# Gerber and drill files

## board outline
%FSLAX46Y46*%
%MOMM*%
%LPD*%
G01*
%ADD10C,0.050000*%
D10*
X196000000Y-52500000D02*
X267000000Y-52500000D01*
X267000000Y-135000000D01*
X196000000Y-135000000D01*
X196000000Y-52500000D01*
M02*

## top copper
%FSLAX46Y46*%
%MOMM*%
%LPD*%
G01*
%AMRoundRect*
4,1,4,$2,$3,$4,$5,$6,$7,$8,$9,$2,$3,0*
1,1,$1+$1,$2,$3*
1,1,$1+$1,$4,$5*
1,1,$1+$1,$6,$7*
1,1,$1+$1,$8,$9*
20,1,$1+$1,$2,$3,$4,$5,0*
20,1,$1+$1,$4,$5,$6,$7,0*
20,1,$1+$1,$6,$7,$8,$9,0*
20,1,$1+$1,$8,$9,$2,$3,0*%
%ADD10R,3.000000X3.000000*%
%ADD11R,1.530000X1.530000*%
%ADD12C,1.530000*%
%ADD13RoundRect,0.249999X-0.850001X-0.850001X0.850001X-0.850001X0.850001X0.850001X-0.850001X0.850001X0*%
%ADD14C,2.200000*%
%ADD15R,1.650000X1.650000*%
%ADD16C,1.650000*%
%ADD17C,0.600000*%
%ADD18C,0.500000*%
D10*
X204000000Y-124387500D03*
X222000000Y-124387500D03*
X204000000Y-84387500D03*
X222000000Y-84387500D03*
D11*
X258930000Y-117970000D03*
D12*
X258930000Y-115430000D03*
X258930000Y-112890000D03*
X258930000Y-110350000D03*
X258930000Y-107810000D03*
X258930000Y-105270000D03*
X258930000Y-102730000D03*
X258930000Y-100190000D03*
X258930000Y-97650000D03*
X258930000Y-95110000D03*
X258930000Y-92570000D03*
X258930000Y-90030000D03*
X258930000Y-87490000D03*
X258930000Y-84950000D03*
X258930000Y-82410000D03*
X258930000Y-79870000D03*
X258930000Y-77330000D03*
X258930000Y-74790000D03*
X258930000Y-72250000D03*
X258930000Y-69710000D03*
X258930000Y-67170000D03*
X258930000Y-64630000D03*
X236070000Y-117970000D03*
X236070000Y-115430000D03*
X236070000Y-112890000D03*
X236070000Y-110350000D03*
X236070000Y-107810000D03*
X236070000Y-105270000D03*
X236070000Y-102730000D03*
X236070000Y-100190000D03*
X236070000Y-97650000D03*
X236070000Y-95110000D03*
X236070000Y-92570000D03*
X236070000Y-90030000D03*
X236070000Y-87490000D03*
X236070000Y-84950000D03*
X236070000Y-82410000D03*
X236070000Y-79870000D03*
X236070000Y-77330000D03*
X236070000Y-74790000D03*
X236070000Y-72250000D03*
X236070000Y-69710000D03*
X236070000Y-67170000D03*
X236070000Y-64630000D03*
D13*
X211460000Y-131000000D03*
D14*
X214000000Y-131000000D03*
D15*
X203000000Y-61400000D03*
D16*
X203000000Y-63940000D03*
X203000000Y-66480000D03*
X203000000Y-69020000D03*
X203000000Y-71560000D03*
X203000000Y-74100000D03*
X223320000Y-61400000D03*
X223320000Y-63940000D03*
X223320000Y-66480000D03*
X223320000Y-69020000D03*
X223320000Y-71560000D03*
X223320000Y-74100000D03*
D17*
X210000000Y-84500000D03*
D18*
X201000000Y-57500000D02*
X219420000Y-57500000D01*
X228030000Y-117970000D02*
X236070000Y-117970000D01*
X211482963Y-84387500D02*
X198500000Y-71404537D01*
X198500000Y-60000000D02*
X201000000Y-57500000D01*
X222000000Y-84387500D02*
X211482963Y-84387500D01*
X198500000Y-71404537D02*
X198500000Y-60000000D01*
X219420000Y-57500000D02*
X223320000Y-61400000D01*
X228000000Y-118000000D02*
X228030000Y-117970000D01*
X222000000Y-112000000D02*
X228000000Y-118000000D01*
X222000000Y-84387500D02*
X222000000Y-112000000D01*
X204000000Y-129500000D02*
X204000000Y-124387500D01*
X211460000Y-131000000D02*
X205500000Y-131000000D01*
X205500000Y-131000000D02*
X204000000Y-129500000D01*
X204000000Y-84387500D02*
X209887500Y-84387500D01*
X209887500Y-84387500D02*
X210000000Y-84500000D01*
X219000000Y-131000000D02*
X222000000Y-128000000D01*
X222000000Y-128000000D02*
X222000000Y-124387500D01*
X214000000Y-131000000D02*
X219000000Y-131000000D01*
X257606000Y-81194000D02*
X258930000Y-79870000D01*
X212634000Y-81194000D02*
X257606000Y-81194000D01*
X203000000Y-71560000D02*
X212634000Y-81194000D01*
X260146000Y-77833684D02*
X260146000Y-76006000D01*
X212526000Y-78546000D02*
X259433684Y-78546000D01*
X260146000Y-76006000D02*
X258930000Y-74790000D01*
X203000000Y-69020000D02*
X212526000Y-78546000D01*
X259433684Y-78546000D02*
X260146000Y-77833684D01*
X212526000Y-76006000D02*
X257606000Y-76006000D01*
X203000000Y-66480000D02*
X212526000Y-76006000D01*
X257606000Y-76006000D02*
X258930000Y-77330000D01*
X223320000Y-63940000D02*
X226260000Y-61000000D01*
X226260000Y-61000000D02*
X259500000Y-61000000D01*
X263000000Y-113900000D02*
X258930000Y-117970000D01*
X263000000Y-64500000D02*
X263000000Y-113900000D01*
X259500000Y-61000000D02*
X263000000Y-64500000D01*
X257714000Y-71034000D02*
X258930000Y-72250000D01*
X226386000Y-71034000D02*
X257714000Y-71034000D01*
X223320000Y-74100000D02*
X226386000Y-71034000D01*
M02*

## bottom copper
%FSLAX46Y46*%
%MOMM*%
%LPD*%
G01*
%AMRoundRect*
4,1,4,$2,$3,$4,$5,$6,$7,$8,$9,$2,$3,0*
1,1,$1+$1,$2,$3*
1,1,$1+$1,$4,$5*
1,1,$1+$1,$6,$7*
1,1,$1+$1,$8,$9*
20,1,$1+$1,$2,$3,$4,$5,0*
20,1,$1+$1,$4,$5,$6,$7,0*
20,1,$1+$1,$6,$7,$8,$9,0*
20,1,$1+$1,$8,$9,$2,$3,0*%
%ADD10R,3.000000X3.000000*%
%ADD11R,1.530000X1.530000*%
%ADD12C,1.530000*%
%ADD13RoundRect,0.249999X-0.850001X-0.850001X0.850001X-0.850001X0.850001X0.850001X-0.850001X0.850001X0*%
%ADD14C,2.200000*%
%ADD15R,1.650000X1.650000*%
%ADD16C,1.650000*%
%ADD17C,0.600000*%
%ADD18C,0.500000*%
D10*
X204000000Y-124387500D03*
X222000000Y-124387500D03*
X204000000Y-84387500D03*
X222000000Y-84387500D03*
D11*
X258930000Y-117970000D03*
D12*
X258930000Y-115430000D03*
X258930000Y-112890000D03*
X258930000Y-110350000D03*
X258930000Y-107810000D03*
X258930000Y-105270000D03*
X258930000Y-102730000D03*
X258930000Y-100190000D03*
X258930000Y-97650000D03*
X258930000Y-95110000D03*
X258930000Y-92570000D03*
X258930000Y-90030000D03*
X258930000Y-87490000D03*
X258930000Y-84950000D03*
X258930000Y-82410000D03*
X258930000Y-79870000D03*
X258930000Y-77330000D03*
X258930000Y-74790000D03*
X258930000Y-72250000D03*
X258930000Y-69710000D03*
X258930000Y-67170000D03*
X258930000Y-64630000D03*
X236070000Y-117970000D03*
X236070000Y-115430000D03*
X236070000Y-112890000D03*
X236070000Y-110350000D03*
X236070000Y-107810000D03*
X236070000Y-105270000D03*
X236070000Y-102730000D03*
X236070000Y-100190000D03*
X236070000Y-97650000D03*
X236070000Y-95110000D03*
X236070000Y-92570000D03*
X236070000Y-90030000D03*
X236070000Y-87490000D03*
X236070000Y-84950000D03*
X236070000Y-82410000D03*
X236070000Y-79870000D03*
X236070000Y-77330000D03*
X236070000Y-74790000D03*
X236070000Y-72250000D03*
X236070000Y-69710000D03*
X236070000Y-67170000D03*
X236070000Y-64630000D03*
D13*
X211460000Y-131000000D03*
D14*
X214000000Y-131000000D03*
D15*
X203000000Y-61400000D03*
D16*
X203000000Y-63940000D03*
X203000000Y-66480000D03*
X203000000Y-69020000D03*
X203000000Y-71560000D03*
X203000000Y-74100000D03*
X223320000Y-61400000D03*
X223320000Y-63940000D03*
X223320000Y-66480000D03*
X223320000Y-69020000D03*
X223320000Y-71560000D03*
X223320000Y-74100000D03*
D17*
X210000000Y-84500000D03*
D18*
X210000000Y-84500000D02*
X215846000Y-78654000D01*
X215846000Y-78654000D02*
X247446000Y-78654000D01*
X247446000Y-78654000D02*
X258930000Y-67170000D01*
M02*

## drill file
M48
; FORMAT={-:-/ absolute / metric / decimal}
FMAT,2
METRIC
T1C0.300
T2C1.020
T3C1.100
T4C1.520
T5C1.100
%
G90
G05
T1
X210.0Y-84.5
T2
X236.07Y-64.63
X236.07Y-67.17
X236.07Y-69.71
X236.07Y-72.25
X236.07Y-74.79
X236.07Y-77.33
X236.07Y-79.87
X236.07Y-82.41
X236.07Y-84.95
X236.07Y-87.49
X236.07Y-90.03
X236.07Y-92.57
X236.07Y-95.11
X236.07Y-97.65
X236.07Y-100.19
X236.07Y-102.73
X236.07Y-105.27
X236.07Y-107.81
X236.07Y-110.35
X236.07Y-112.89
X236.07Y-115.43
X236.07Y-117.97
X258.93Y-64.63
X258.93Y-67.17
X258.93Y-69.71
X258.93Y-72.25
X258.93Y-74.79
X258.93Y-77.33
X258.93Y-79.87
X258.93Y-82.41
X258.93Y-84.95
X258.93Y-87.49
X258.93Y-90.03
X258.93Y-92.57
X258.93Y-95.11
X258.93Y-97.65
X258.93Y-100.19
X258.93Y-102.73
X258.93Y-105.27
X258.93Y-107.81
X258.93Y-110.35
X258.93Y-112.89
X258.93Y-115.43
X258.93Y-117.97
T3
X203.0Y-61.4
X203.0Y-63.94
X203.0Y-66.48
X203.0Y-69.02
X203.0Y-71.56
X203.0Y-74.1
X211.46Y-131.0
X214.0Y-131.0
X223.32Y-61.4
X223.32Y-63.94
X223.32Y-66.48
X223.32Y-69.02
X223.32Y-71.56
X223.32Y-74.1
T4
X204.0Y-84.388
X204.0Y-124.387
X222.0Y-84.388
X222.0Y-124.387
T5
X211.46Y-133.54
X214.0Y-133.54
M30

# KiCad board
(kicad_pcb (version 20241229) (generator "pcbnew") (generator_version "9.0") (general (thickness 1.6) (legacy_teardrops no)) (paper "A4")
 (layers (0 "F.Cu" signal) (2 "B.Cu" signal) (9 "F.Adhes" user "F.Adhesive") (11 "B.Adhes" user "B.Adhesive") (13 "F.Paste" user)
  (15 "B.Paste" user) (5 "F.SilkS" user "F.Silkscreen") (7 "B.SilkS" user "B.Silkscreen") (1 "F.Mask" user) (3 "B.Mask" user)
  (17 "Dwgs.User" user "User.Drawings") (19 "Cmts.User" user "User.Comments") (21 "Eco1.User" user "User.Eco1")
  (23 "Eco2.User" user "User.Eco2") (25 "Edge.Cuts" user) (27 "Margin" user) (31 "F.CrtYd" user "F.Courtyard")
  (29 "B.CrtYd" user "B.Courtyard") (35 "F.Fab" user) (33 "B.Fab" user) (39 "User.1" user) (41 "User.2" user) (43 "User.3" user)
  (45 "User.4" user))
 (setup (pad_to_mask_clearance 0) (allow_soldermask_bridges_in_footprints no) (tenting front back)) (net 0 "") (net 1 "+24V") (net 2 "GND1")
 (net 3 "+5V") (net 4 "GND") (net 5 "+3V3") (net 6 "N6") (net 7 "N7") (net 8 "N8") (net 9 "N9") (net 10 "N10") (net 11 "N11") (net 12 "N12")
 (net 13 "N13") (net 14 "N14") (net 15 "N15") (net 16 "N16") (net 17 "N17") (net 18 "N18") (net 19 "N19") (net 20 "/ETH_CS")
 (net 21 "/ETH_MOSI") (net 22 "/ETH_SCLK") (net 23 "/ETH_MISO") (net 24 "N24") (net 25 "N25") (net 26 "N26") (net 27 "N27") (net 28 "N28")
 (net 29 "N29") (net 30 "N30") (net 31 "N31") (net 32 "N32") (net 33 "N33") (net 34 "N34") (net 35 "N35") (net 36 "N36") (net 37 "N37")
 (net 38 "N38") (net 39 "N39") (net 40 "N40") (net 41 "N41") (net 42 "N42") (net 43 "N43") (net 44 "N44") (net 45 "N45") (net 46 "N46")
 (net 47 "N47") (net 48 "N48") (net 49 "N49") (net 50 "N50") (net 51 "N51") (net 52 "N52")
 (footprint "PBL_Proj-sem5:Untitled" (layer "F.Cu") (at 201.5 126.8875 90)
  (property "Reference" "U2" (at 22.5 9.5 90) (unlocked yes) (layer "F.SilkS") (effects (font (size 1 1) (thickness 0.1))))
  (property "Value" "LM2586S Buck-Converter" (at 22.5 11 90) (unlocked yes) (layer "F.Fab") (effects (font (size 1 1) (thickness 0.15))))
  (pad "1" thru_hole rect (at 2.5 2.5 90) (size 3 3) (drill 1.52) (layers "*.Cu" "*.Mask") (remove_unused_layers no) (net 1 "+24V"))
  (pad "2" thru_hole rect (at 2.5 20.5 90) (size 3 3) (drill 1.52) (layers "*.Cu" "*.Mask") (remove_unused_layers no) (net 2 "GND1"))
  (pad "3" thru_hole rect (at 42.5 2.5 90) (size 3 3) (drill 1.52) (layers "*.Cu" "*.Mask") (remove_unused_layers no) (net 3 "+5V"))
  (pad "4" thru_hole rect (at 42.5 20.5 90) (size 3 3) (drill 1.52) (layers "*.Cu" "*.Mask") (remove_unused_layers no) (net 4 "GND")))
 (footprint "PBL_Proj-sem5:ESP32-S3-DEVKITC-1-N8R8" (layer "F.Cu") (at 247.5 88 180)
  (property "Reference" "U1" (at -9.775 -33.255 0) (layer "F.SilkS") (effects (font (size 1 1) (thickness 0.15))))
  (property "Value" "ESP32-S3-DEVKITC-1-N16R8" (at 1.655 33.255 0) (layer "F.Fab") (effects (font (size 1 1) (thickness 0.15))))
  (pad "J1_1" thru_hole rect (at -11.43 -29.97 180) (size 1.53 1.53) (drill 1.02) (layers "*.Cu" "*.Mask") (remove_unused_layers no)
   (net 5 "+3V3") (solder_mask_margin 0.102))
  (pad "J1_2" thru_hole circle (at -11.43 -27.43 180) (size 1.53 1.53) (drill 1.02) (layers "*.Cu" "*.Mask") (remove_unused_layers no)
   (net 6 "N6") (solder_mask_margin 0.102))
  (pad "J1_3" thru_hole circle (at -11.43 -24.89 180) (size 1.53 1.53) (drill 1.02) (layers "*.Cu" "*.Mask") (remove_unused_layers no)
   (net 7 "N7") (solder_mask_margin 0.102))
  (pad "J1_4" thru_hole circle (at -11.43 -22.35 180) (size 1.53 1.53) (drill 1.02) (layers "*.Cu" "*.Mask") (remove_unused_layers no)
   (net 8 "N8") (solder_mask_margin 0.102))
  (pad "J1_5" thru_hole circle (at -11.43 -19.81 180) (size 1.53 1.53) (drill 1.02) (layers "*.Cu" "*.Mask") (remove_unused_layers no)
   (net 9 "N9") (solder_mask_margin 0.102))
  (pad "J1_6" thru_hole circle (at -11.43 -17.27 180) (size 1.53 1.53) (drill 1.02) (layers "*.Cu" "*.Mask") (remove_unused_layers no)
   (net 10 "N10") (solder_mask_margin 0.102))
  (pad "J1_7" thru_hole circle (at -11.43 -14.73 180) (size 1.53 1.53) (drill 1.02) (layers "*.Cu" "*.Mask") (remove_unused_layers no)
   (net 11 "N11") (solder_mask_margin 0.102))
  (pad "J1_8" thru_hole circle (at -11.43 -12.19 180) (size 1.53 1.53) (drill 1.02) (layers "*.Cu" "*.Mask") (remove_unused_layers no)
   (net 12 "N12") (solder_mask_margin 0.102))
  (pad "J1_9" thru_hole circle (at -11.43 -9.65 180) (size 1.53 1.53) (drill 1.02) (layers "*.Cu" "*.Mask") (remove_unused_layers no)
   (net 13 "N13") (solder_mask_margin 0.102))
  (pad "J1_10" thru_hole circle (at -11.43 -7.11 180) (size 1.53 1.53) (drill 1.02) (layers "*.Cu" "*.Mask") (remove_unused_layers no)
   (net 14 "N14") (solder_mask_margin 0.102))
  (pad "J1_11" thru_hole circle (at -11.43 -4.57 180) (size 1.53 1.53) (drill 1.02) (layers "*.Cu" "*.Mask") (remove_unused_layers no)
   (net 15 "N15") (solder_mask_margin 0.102))
  (pad "J1_12" thru_hole circle (at -11.43 -2.03 180) (size 1.53 1.53) (drill 1.02) (layers "*.Cu" "*.Mask") (remove_unused_layers no)
   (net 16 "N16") (solder_mask_margin 0.102))
  (pad "J1_13" thru_hole circle (at -11.43 0.51 180) (size 1.53 1.53) (drill 1.02) (layers "*.Cu" "*.Mask") (remove_unused_layers no)
   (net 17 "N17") (solder_mask_margin 0.102))
  (pad "J1_14" thru_hole circle (at -11.43 3.05 180) (size 1.53 1.53) (drill 1.02) (layers "*.Cu" "*.Mask") (remove_unused_layers no)
   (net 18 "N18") (solder_mask_margin 0.102))
  (pad "J1_15" thru_hole circle (at -11.43 5.59 180) (size 1.53 1.53) (drill 1.02) (layers "*.Cu" "*.Mask") (remove_unused_layers no)
   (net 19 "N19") (solder_mask_margin 0.102))
  (pad "J1_16" thru_hole circle (at -11.43 8.13 180) (size 1.53 1.53) (drill 1.02) (layers "*.Cu" "*.Mask") (remove_unused_layers no)
   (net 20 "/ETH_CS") (solder_mask_margin 0.102))
  (pad "J1_17" thru_hole circle (at -11.43 10.67 180) (size 1.53 1.53) (drill 1.02) (layers "*.Cu" "*.Mask") (remove_unused_layers no)
   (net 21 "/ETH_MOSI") (solder_mask_margin 0.102))
  (pad "J1_18" thru_hole circle (at -11.43 13.21 180) (size 1.53 1.53) (drill 1.02) (layers "*.Cu" "*.Mask") (remove_unused_layers no)
   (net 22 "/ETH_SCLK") (solder_mask_margin 0.102))
  (pad "J1_19" thru_hole circle (at -11.43 15.75 180) (size 1.53 1.53) (drill 1.02) (layers "*.Cu" "*.Mask") (remove_unused_layers no)
   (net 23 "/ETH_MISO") (solder_mask_margin 0.102))
  (pad "J1_20" thru_hole circle (at -11.43 18.29 180) (size 1.53 1.53) (drill 1.02) (layers "*.Cu" "*.Mask") (remove_unused_layers no)
   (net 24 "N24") (solder_mask_margin 0.102))
  (pad "J1_21" thru_hole circle (at -11.43 20.83 180) (size 1.53 1.53) (drill 1.02) (layers "*.Cu" "*.Mask") (remove_unused_layers no)
   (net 3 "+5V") (solder_mask_margin 0.102))
  (pad "J1_22" thru_hole circle (at -11.43 23.37 180) (size 1.53 1.53) (drill 1.02) (layers "*.Cu" "*.Mask") (remove_unused_layers no)
   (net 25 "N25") (solder_mask_margin 0.102))
  (pad "J3_1" thru_hole circle (at 11.43 -29.97 180) (size 1.53 1.53) (drill 1.02) (layers "*.Cu" "*.Mask") (remove_unused_layers no)
   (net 4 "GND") (solder_mask_margin 0.102))
  (pad "J3_2" thru_hole circle (at 11.43 -27.43 180) (size 1.53 1.53) (drill 1.02) (layers "*.Cu" "*.Mask") (remove_unused_layers no)
   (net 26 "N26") (solder_mask_margin 0.102))
  (pad "J3_3" thru_hole circle (at 11.43 -24.89 180) (size 1.53 1.53) (drill 1.02) (layers "*.Cu" "*.Mask") (remove_unused_layers no)
   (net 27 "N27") (solder_mask_margin 0.102))
  (pad "J3_4" thru_hole circle (at 11.43 -22.35 180) (size 1.53 1.53) (drill 1.02) (layers "*.Cu" "*.Mask") (remove_unused_layers no)
   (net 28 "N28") (solder_mask_margin 0.102))
  (pad "J3_5" thru_hole circle (at 11.43 -19.81 180) (size 1.53 1.53) (drill 1.02) (layers "*.Cu" "*.Mask") (remove_unused_layers no)
   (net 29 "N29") (solder_mask_margin 0.102))
  (pad "J3_6" thru_hole circle (at 11.43 -17.27 180) (size 1.53 1.53) (drill 1.02) (layers "*.Cu" "*.Mask") (remove_unused_layers no)
   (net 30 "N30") (solder_mask_margin 0.102))
  (pad "J3_7" thru_hole circle (at 11.43 -14.73 180) (size 1.53 1.53) (drill 1.02) (layers "*.Cu" "*.Mask") (remove_unused_layers no)
   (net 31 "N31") (solder_mask_margin 0.102))
  (pad "J3_8" thru_hole circle (at 11.43 -12.19 180) (size 1.53 1.53) (drill 1.02) (layers "*.Cu" "*.Mask") (remove_unused_layers no)
   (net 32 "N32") (solder_mask_margin 0.102))
  (pad "J3_9" thru_hole circle (at 11.43 -9.65 180) (size 1.53 1.53) (drill 1.02) (layers "*.Cu" "*.Mask") (remove_unused_layers no)
   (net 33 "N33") (solder_mask_margin 0.102))
  (pad "J3_10" thru_hole circle (at 11.43 -7.11 180) (size 1.53 1.53) (drill 1.02) (layers "*.Cu" "*.Mask") (remove_unused_layers no)
   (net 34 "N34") (solder_mask_margin 0.102))
  (pad "J3_11" thru_hole circle (at 11.43 -4.57 180) (size 1.53 1.53) (drill 1.02) (layers "*.Cu" "*.Mask") (remove_unused_layers no)
   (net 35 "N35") (solder_mask_margin 0.102))
  (pad "J3_12" thru_hole circle (at 11.43 -2.03 180) (size 1.53 1.53) (drill 1.02) (layers "*.Cu" "*.Mask") (remove_unused_layers no)
   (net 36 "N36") (solder_mask_margin 0.102))
  (pad "J3_13" thru_hole circle (at 11.43 0.51 180) (size 1.53 1.53) (drill 1.02) (layers "*.Cu" "*.Mask") (remove_unused_layers no)
   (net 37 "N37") (solder_mask_margin 0.102))
  (pad "J3_14" thru_hole circle (at 11.43 3.05 180) (size 1.53 1.53) (drill 1.02) (layers "*.Cu" "*.Mask") (remove_unused_layers no)
   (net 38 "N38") (solder_mask_margin 0.102))
  (pad "J3_15" thru_hole circle (at 11.43 5.59 180) (size 1.53 1.53) (drill 1.02) (layers "*.Cu" "*.Mask") (remove_unused_layers no)
   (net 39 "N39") (solder_mask_margin 0.102))
  (pad "J3_16" thru_hole circle (at 11.43 8.13 180) (size 1.53 1.53) (drill 1.02) (layers "*.Cu" "*.Mask") (remove_unused_layers no)
   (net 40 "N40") (solder_mask_margin 0.102))
  (pad "J3_17" thru_hole circle (at 11.43 10.67 180) (size 1.53 1.53) (drill 1.02) (layers "*.Cu" "*.Mask") (remove_unused_layers no)
   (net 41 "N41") (solder_mask_margin 0.102))
  (pad "J3_18" thru_hole circle (at 11.43 13.21 180) (size 1.53 1.53) (drill 1.02) (layers "*.Cu" "*.Mask") (remove_unused_layers no)
   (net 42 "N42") (solder_mask_margin 0.102))
  (pad "J3_19" thru_hole circle (at 11.43 15.75 180) (size 1.53 1.53) (drill 1.02) (layers "*.Cu" "*.Mask") (remove_unused_layers no)
   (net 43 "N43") (solder_mask_margin 0.102))
  (pad "J3_20" thru_hole circle (at 11.43 18.29 180) (size 1.53 1.53) (drill 1.02) (layers "*.Cu" "*.Mask") (remove_unused_layers no)
   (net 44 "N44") (solder_mask_margin 0.102))
  (pad "J3_21" thru_hole circle (at 11.43 20.83 180) (size 1.53 1.53) (drill 1.02) (layers "*.Cu" "*.Mask") (remove_unused_layers no)
   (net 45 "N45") (solder_mask_margin 0.102))
  (pad "J3_22" thru_hole circle (at 11.43 23.37 180) (size 1.53 1.53) (drill 1.02) (layers "*.Cu" "*.Mask") (remove_unused_layers no)
   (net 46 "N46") (solder_mask_margin 0.102)))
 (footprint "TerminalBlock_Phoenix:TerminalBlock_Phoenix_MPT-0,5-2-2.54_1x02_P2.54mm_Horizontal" (layer "F.Cu") (at 211.46 131)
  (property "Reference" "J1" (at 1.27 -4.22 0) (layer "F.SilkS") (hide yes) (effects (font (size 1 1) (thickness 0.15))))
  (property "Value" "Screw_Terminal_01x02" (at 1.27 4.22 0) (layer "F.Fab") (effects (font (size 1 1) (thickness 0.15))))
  (pad "" np_thru_hole circle (at 0 2.54) (size 1.1 1.1) (drill 1.1) (layers "*.Cu" "*.Mask"))
  (pad "" np_thru_hole circle (at 2.54 2.54) (size 1.1 1.1) (drill 1.1) (layers "*.Cu" "*.Mask"))
  (pad "1" thru_hole roundrect (at 0 0) (size 2.2 2.2) (drill 1.1) (layers "*.Cu" "*.Mask") (remove_unused_layers no)
   (roundrect_rratio 0.113636) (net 1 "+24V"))
  (pad "2" thru_hole circle (at 2.54 0) (size 2.2 2.2) (drill 1.1) (layers "*.Cu" "*.Mask") (remove_unused_layers no) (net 2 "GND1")))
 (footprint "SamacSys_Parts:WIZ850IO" (layer "F.Cu") (at 203 61.4)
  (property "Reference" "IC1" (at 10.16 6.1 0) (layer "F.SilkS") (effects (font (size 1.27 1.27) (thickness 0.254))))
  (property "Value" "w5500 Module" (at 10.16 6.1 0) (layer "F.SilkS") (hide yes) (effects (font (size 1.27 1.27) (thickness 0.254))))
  (pad "J11" thru_hole rect (at 0 0) (size 1.65 1.65) (drill 1.1) (layers "*.Cu" "*.Mask") (remove_unused_layers no) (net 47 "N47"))
  (pad "J12" thru_hole circle (at 0 2.54) (size 1.65 1.65) (drill 1.1) (layers "*.Cu" "*.Mask") (remove_unused_layers no) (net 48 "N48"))
  (pad "J13" thru_hole circle (at 0 5.08) (size 1.65 1.65) (drill 1.1) (layers "*.Cu" "*.Mask") (remove_unused_layers no)
   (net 21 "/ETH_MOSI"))
  (pad "J14" thru_hole circle (at 0 7.62) (size 1.65 1.65) (drill 1.1) (layers "*.Cu" "*.Mask") (remove_unused_layers no)
   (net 22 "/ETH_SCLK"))
  (pad "J15" thru_hole circle (at 0 10.16) (size 1.65 1.65) (drill 1.1) (layers "*.Cu" "*.Mask") (remove_unused_layers no)
   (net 20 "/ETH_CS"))
  (pad "J16" thru_hole circle (at 0 12.7) (size 1.65 1.65) (drill 1.1) (layers "*.Cu" "*.Mask") (remove_unused_layers no) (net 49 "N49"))
  (pad "J21" thru_hole circle (at 20.32 0) (size 1.65 1.65) (drill 1.1) (layers "*.Cu" "*.Mask") (remove_unused_layers no) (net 4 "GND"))
  (pad "J22" thru_hole circle (at 20.32 2.54) (size 1.65 1.65) (drill 1.1) (layers "*.Cu" "*.Mask") (remove_unused_layers no) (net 5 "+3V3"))
  (pad "J23" thru_hole circle (at 20.32 5.08) (size 1.65 1.65) (drill 1.1) (layers "*.Cu" "*.Mask") (remove_unused_layers no) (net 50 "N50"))
  (pad "J24" thru_hole circle (at 20.32 7.62) (size 1.65 1.65) (drill 1.1) (layers "*.Cu" "*.Mask") (remove_unused_layers no) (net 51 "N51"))
  (pad "J25" thru_hole circle (at 20.32 10.16) (size 1.65 1.65) (drill 1.1) (layers "*.Cu" "*.Mask") (remove_unused_layers no)
   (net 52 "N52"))
  (pad "J26" thru_hole circle (at 20.32 12.7) (size 1.65 1.65) (drill 1.1) (layers "*.Cu" "*.Mask") (remove_unused_layers no)
   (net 23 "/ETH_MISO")))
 (gr_rect (start 196 52.5) (end 267 135) (stroke (width 0.05) (type default)) (fill no) (layer "Edge.Cuts"))
 (segment (start 201 57.5) (end 219.42 57.5) (width 0.5) (layer "F.Cu") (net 4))
 (segment (start 228.03 117.97) (end 236.07 117.97) (width 0.5) (layer "F.Cu") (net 4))
 (segment (start 211.482963 84.3875) (end 198.5 71.404537) (width 0.5) (layer "F.Cu") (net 4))
 (segment (start 198.5 60) (end 201 57.5) (width 0.5) (layer "F.Cu") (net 4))
 (segment (start 222 84.3875) (end 211.482963 84.3875) (width 0.5) (layer "F.Cu") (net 4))
 (segment (start 198.5 71.404537) (end 198.5 60) (width 0.5) (layer "F.Cu") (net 4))
 (segment (start 219.42 57.5) (end 223.32 61.4) (width 0.5) (layer "F.Cu") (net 4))
 (segment (start 228 118) (end 228.03 117.97) (width 0.5) (layer "F.Cu") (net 4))
 (segment (start 222 112) (end 228 118) (width 0.5) (layer "F.Cu") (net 4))
 (segment (start 222 84.3875) (end 222 112) (width 0.5) (layer "F.Cu") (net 4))
 (segment (start 204 129.5) (end 204 124.3875) (width 0.5) (layer "F.Cu") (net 1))
 (segment (start 211.46 131) (end 205.5 131) (width 0.5) (layer "F.Cu") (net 1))
 (segment (start 205.5 131) (end 204 129.5) (width 0.5) (layer "F.Cu") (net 1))
 (segment (start 204 84.3875) (end 209.8875 84.3875) (width 0.5) (layer "F.Cu") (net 3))
 (segment (start 209.8875 84.3875) (end 210 84.5) (width 0.5) (layer "F.Cu") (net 3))
 (via (at 210 84.5) (size 0.6) (drill 0.3) (layers "F.Cu" "B.Cu") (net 3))
 (segment (start 210 84.5) (end 215.846 78.654) (width 0.5) (layer "B.Cu") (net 3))
 (segment (start 215.846 78.654) (end 247.446 78.654) (width 0.5) (layer "B.Cu") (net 3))
 (segment (start 247.446 78.654) (end 258.93 67.17) (width 0.5) (layer "B.Cu") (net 3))
 (segment (start 219 131) (end 222 128) (width 0.5) (layer "F.Cu") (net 2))
 (segment (start 222 128) (end 222 124.3875) (width 0.5) (layer "F.Cu") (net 2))
 (segment (start 214 131) (end 219 131) (width 0.5) (layer "F.Cu") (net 2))
 (segment (start 257.606 81.194) (end 258.93 79.87) (width 0.5) (layer "F.Cu") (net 20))
 (segment (start 212.634 81.194) (end 257.606 81.194) (width 0.5) (layer "F.Cu") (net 20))
 (segment (start 203 71.56) (end 212.634 81.194) (width 0.5) (layer "F.Cu") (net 20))
 (segment (start 260.146 77.833684) (end 260.146 76.006) (width 0.5) (layer "F.Cu") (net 22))
 (segment (start 212.526 78.546) (end 259.433684 78.546) (width 0.5) (layer "F.Cu") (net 22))
 (segment (start 260.146 76.006) (end 258.93 74.79) (width 0.5) (layer "F.Cu") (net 22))
 (segment (start 203 69.02) (end 212.526 78.546) (width 0.5) (layer "F.Cu") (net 22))
 (segment (start 259.433684 78.546) (end 260.146 77.833684) (width 0.5) (layer "F.Cu") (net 22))
 (segment (start 212.526 76.006) (end 257.606 76.006) (width 0.5) (layer "F.Cu") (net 21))
 (segment (start 203 66.48) (end 212.526 76.006) (width 0.5) (layer "F.Cu") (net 21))
 (segment (start 257.606 76.006) (end 258.93 77.33) (width 0.5) (layer "F.Cu") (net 21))
 (segment (start 223.32 63.94) (end 226.26 61) (width 0.5) (layer "F.Cu") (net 5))
 (segment (start 226.26 61) (end 259.5 61) (width 0.5) (layer "F.Cu") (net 5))
 (segment (start 263 113.9) (end 258.93 117.97) (width 0.5) (layer "F.Cu") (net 5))
 (segment (start 263 64.5) (end 263 113.9) (width 0.5) (layer "F.Cu") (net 5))
 (segment (start 259.5 61) (end 263 64.5) (width 0.5) (layer "F.Cu") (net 5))
 (segment (start 257.714 71.034) (end 258.93 72.25) (width 0.5) (layer "F.Cu") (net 23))
 (segment (start 226.386 71.034) (end 257.714 71.034) (width 0.5) (layer "F.Cu") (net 23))
 (segment (start 223.32 74.1) (end 226.386 71.034) (width 0.5) (layer "F.Cu") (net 23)))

